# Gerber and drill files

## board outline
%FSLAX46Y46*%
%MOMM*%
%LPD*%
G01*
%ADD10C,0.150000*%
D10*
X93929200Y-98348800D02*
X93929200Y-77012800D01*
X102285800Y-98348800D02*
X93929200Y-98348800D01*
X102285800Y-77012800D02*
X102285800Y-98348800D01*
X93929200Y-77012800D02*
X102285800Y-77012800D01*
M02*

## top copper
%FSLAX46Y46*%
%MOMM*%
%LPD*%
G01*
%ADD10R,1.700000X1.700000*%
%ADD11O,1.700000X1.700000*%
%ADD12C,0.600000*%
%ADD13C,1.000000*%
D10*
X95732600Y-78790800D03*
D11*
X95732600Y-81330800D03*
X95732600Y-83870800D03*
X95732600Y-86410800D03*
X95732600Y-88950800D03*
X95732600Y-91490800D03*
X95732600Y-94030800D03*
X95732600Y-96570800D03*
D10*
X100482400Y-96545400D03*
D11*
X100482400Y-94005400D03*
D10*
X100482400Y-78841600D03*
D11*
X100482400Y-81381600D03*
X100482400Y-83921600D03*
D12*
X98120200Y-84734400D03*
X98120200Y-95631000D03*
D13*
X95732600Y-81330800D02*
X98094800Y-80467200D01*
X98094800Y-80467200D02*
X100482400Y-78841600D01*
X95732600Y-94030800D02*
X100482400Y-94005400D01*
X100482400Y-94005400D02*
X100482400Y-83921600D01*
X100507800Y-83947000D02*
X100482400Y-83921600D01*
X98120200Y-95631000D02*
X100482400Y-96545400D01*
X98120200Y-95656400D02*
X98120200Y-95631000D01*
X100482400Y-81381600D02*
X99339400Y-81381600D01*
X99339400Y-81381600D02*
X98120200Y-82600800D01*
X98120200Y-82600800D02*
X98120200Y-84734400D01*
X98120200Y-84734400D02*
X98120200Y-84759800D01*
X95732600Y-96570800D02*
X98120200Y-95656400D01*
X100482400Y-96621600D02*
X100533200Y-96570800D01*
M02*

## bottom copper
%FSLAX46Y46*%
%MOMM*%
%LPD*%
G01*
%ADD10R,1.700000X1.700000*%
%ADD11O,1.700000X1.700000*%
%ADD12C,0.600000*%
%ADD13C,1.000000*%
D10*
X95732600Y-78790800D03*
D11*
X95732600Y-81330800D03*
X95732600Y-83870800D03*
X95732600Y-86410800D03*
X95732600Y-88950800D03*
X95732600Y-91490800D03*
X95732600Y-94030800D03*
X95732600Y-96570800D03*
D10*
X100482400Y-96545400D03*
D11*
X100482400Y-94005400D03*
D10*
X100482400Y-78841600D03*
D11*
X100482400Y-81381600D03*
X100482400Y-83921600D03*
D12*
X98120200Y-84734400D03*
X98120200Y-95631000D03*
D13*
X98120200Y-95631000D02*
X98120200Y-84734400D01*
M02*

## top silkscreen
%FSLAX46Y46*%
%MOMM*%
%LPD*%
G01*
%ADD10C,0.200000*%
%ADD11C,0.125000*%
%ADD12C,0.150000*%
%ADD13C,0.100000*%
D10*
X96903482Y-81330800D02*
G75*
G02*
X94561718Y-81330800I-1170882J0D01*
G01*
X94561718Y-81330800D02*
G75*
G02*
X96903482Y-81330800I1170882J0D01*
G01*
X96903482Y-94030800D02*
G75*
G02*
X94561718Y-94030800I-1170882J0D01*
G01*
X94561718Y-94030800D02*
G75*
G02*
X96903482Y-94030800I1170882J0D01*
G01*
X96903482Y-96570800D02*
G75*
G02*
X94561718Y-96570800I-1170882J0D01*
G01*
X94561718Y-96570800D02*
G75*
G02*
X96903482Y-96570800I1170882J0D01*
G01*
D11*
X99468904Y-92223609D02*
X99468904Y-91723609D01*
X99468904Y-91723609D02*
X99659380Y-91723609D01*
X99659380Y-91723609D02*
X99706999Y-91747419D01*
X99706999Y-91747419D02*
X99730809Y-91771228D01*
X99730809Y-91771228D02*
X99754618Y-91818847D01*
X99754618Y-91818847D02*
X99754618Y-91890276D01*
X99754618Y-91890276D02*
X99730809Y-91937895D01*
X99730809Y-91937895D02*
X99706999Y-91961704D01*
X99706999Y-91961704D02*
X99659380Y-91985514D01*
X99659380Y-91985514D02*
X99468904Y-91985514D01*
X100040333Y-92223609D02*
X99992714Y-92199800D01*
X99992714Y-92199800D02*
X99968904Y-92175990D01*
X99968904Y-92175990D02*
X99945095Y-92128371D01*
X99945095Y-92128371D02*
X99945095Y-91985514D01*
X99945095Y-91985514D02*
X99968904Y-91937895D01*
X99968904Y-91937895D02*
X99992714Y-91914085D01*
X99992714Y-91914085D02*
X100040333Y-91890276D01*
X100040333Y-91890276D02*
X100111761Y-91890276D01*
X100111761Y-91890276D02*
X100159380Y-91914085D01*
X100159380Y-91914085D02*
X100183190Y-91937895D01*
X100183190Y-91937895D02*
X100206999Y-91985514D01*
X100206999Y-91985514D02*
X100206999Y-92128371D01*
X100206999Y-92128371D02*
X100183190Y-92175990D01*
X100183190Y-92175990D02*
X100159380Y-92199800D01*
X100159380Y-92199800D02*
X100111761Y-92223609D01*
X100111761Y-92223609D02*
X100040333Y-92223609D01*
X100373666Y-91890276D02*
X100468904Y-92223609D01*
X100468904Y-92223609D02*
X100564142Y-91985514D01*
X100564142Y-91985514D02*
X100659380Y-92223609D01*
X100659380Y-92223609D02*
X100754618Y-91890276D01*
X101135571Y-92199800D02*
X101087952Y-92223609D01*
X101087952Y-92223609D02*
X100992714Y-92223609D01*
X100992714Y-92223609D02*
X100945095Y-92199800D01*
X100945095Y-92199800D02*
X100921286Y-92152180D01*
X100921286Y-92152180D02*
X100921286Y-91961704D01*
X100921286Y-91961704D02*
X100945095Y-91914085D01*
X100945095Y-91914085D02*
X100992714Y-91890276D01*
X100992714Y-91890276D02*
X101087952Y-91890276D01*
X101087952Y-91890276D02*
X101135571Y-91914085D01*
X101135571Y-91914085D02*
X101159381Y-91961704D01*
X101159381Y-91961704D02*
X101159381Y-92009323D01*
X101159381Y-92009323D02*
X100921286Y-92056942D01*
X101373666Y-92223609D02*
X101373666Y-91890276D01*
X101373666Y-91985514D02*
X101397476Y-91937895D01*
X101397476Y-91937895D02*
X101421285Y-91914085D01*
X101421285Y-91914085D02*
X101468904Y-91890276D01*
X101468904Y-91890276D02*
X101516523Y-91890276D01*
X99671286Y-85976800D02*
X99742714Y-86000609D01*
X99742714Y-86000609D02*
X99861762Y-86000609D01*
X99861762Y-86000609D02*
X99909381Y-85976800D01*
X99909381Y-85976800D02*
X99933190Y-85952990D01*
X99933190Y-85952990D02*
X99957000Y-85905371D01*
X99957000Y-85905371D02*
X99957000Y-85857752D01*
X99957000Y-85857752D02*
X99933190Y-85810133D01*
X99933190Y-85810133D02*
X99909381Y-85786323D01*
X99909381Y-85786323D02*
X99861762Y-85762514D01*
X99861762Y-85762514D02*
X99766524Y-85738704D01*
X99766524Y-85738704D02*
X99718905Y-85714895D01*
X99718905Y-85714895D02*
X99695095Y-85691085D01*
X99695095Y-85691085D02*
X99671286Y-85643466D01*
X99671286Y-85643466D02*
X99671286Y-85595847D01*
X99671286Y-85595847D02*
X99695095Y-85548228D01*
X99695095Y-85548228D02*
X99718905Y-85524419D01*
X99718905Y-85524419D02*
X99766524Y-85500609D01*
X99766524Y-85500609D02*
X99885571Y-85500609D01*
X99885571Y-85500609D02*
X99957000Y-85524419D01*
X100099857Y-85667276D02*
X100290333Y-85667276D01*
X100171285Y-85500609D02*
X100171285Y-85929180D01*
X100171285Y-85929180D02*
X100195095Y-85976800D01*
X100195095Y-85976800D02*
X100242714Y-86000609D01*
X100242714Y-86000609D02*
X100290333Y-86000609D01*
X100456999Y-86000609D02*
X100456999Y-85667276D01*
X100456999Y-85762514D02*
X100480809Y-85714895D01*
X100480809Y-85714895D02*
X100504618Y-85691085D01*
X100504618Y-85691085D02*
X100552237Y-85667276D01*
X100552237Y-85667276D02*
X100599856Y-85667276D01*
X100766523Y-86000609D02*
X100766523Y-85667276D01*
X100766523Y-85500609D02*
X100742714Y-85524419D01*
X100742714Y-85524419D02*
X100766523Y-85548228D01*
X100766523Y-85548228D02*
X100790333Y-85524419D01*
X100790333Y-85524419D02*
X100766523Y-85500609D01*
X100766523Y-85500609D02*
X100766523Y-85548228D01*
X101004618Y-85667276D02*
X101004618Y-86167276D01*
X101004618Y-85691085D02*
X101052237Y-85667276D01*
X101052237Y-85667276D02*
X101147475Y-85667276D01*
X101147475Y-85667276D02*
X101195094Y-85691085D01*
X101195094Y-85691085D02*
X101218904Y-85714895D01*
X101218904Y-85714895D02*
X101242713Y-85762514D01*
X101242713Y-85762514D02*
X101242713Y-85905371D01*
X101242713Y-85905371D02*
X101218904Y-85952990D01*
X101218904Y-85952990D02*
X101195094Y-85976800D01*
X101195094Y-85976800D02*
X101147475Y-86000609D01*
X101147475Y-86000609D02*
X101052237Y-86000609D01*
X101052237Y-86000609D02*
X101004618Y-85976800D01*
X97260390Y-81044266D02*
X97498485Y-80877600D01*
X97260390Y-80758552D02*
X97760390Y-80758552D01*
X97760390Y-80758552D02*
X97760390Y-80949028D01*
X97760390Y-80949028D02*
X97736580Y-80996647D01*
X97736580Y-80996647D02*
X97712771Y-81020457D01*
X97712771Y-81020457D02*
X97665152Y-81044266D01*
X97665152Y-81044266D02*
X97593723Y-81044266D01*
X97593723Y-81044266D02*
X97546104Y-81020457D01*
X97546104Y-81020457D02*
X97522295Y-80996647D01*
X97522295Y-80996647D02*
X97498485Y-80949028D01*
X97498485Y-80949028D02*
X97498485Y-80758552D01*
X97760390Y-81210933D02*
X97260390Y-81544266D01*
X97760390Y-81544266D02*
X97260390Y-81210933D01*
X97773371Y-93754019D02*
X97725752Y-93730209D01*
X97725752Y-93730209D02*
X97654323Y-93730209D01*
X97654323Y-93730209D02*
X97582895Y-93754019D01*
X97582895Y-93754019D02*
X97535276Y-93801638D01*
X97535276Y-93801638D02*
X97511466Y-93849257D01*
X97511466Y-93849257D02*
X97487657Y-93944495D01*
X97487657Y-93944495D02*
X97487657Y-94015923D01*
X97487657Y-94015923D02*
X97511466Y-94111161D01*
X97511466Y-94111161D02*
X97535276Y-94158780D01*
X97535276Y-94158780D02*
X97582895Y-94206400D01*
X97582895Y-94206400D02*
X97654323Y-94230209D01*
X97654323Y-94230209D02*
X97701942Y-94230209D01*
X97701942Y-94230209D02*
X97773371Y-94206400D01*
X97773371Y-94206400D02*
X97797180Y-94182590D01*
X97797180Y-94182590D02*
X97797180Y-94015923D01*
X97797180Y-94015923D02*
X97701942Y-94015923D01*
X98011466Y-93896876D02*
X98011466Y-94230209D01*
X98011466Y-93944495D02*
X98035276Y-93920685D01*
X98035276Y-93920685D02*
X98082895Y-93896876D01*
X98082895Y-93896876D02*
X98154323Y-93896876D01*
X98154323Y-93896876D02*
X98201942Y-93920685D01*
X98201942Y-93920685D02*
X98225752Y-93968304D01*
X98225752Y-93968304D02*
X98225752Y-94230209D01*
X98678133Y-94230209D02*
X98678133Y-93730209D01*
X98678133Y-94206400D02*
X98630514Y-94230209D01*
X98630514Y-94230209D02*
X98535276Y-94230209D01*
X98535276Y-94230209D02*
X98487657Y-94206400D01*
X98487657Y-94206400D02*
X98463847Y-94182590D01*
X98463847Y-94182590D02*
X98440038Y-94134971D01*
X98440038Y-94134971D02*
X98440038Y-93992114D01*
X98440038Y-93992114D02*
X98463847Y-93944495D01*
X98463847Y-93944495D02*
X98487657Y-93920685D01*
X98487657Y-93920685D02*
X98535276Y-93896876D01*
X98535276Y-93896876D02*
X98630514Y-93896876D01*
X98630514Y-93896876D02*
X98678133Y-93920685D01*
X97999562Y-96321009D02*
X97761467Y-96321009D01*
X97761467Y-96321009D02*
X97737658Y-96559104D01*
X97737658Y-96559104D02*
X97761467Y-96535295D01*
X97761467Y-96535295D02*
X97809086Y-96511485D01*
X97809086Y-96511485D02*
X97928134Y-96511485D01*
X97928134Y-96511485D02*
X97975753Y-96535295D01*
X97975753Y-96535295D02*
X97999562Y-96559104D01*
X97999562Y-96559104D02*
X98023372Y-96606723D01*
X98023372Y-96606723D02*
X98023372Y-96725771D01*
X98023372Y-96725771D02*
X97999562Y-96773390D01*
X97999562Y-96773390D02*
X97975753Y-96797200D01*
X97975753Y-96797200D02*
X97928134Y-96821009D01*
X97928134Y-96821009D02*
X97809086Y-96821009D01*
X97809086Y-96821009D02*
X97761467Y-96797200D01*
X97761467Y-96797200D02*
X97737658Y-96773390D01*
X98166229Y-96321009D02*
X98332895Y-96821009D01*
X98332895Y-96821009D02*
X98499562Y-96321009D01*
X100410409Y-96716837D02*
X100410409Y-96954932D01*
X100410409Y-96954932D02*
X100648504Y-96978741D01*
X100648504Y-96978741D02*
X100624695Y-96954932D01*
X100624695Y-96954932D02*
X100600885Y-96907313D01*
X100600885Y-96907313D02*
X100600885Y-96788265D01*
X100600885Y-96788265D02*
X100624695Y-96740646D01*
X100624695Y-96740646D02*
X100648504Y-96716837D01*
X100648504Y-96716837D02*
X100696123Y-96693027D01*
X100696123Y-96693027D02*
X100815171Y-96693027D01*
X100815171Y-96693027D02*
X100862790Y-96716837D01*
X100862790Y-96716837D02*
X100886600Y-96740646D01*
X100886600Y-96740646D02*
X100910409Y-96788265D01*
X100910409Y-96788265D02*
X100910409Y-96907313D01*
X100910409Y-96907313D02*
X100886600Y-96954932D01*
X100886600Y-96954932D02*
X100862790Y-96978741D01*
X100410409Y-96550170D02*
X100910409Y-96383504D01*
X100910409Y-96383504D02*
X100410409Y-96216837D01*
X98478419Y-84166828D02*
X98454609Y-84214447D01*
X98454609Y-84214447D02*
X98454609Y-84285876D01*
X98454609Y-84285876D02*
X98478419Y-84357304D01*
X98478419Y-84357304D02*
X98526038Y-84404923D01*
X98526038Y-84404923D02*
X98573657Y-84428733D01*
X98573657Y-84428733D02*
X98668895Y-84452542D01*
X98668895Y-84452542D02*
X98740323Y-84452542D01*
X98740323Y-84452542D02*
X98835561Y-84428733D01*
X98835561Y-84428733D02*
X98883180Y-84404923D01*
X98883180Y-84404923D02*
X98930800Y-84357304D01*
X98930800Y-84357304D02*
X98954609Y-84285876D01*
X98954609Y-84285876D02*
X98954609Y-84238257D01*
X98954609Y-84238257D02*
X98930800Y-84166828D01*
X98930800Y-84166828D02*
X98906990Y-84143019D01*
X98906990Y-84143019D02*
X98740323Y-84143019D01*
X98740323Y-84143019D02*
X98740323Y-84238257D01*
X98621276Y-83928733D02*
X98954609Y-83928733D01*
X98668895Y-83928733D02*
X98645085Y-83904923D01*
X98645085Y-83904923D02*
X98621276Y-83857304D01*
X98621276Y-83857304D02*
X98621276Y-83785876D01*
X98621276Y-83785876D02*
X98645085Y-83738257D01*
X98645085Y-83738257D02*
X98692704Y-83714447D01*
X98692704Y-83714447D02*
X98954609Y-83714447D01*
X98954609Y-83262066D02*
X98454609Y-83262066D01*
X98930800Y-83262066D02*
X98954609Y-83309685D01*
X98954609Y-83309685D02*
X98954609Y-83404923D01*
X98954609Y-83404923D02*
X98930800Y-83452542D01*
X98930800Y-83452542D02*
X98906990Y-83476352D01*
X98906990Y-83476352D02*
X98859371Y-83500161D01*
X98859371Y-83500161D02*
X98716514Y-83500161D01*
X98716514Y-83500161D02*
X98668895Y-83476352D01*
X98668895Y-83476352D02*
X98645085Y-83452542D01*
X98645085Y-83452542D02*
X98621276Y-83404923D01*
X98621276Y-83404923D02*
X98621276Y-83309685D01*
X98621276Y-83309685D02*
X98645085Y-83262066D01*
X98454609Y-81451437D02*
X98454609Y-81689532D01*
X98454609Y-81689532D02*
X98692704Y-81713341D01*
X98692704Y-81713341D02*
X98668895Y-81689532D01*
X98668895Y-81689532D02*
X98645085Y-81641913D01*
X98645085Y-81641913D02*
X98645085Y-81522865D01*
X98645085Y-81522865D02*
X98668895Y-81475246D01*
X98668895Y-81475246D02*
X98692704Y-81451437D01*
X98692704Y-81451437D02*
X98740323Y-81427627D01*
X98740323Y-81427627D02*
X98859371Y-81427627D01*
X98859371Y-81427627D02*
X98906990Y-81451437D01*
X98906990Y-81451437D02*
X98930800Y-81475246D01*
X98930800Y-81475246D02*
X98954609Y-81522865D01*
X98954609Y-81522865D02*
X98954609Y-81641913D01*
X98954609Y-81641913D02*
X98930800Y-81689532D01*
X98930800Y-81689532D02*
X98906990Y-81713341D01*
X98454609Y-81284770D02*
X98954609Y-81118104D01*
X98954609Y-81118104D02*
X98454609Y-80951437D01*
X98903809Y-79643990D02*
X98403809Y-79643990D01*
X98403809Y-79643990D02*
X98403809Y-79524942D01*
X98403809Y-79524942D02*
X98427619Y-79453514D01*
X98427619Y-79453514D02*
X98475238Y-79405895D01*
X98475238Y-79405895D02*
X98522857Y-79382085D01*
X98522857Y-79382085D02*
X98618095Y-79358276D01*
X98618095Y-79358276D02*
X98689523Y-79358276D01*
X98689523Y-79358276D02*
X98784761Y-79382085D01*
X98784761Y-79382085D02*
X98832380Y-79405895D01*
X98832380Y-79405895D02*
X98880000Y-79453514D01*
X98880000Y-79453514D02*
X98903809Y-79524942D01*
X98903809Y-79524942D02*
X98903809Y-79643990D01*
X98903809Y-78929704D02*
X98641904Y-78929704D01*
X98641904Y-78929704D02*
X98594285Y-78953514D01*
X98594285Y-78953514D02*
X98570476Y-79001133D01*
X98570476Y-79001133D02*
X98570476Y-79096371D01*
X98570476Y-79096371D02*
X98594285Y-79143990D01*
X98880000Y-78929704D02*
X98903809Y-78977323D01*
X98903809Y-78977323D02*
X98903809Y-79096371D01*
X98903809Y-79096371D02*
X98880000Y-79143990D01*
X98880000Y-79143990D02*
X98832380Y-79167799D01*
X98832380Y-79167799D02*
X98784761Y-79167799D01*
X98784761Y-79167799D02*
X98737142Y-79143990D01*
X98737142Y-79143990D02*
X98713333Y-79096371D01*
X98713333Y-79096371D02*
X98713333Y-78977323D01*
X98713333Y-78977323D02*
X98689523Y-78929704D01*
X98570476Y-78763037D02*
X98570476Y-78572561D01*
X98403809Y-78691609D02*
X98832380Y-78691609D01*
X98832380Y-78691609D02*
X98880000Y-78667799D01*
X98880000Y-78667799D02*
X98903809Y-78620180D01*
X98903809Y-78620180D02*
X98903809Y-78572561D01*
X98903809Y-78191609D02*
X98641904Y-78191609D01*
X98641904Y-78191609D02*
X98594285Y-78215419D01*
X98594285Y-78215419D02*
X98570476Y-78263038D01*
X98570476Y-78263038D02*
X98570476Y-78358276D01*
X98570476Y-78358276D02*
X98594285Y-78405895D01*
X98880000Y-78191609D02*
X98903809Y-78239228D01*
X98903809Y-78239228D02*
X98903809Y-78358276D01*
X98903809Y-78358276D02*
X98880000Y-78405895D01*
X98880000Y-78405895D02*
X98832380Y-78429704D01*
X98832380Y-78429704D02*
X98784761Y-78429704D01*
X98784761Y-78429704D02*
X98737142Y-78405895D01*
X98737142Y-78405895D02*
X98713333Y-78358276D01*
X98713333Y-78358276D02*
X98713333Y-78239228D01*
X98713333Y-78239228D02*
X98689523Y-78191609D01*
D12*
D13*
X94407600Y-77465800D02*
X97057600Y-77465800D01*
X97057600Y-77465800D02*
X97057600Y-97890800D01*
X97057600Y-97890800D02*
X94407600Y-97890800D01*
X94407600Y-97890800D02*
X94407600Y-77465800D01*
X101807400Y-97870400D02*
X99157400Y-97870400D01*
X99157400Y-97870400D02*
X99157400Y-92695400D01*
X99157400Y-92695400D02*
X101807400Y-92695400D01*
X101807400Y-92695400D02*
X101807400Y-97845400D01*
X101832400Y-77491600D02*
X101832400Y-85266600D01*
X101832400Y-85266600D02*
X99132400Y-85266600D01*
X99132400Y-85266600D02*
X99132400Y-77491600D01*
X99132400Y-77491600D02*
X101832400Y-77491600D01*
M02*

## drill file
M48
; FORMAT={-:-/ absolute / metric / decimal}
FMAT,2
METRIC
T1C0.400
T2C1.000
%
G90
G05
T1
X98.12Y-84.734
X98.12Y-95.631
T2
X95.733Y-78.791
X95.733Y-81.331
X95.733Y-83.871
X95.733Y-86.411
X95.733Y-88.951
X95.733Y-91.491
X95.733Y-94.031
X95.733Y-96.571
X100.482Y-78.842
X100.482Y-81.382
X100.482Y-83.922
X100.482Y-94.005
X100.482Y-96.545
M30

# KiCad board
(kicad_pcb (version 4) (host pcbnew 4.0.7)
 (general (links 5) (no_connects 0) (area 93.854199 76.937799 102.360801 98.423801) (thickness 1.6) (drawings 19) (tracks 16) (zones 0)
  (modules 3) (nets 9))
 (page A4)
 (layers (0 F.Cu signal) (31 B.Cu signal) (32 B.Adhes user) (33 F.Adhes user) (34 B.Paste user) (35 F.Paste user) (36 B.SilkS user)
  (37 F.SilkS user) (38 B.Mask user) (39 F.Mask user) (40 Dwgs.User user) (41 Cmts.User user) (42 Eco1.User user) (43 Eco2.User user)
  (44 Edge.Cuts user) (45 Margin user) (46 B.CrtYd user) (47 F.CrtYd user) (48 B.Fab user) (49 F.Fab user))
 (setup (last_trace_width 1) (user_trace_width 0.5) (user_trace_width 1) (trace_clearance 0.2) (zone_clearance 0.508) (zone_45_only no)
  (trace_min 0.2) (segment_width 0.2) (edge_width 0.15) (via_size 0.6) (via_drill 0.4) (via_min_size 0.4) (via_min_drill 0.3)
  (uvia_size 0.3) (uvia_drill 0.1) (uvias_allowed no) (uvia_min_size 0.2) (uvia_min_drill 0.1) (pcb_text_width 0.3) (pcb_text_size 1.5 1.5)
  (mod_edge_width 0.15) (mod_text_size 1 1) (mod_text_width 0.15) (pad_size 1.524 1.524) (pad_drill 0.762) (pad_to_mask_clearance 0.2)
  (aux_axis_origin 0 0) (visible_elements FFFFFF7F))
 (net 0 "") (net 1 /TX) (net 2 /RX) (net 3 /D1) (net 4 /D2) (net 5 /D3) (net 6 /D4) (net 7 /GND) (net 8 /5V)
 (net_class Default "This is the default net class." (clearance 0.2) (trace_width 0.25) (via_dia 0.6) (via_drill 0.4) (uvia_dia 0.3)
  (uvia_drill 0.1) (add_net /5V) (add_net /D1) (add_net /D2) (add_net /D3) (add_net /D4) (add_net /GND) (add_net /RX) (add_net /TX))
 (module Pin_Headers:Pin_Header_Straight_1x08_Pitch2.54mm (layer F.Cu) (at 95.7326 78.7908)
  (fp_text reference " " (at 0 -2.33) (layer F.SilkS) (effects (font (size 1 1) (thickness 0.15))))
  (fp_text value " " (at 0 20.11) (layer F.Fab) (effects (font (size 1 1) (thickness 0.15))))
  (fp_line (start -1.325 -1.325) (end 1.325 -1.325) (layer F.SilkS) (width 0.1))
  (fp_line (start 1.325 -1.325) (end 1.325 19.1) (layer F.SilkS) (width 0.1))
  (fp_line (start 1.325 19.1) (end -1.325 19.1) (layer F.SilkS) (width 0.1))
  (fp_line (start -1.325 19.1) (end -1.325 -1.325) (layer F.SilkS) (width 0.1))
  (pad 1 thru_hole rect (at 0 0) (size 1.7 1.7) (drill 1) (layers *.Cu *.Mask) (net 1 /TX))
  (pad 2 thru_hole oval (at 0 2.54) (size 1.7 1.7) (drill 1) (layers *.Cu *.Mask) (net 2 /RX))
  (pad 3 thru_hole oval (at 0 5.08) (size 1.7 1.7) (drill 1) (layers *.Cu *.Mask) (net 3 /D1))
  (pad 4 thru_hole oval (at 0 7.62) (size 1.7 1.7) (drill 1) (layers *.Cu *.Mask) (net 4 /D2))
  (pad 5 thru_hole oval (at 0 10.16) (size 1.7 1.7) (drill 1) (layers *.Cu *.Mask) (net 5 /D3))
  (pad 6 thru_hole oval (at 0 12.7) (size 1.7 1.7) (drill 1) (layers *.Cu *.Mask) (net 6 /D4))
  (pad 7 thru_hole oval (at 0 15.24) (size 1.7 1.7) (drill 1) (layers *.Cu *.Mask) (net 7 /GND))
  (pad 8 thru_hole oval (at 0 17.78) (size 1.7 1.7) (drill 1) (layers *.Cu *.Mask) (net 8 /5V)))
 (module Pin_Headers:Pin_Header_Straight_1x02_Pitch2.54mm (layer F.Cu) (at 100.4824 96.5454 180)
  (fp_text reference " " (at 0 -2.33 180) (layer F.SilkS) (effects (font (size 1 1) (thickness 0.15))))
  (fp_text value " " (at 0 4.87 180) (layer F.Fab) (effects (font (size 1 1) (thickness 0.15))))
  (fp_line (start -1.325 -1.325) (end 1.325 -1.325) (layer F.SilkS) (width 0.1))
  (fp_line (start 1.325 -1.325) (end 1.325 3.85) (layer F.SilkS) (width 0.1))
  (fp_line (start 1.325 3.85) (end -1.325 3.85) (layer F.SilkS) (width 0.1))
  (fp_line (start -1.325 3.85) (end -1.325 -1.3) (layer F.SilkS) (width 0.1))
  (pad 1 thru_hole rect (at 0 0 180) (size 1.7 1.7) (drill 1) (layers *.Cu *.Mask) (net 8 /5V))
  (pad 2 thru_hole oval (at 0 2.54 180) (size 1.7 1.7) (drill 1) (layers *.Cu *.Mask) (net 7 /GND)))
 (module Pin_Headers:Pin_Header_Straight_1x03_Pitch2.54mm (layer F.Cu) (at 100.4824 78.8416)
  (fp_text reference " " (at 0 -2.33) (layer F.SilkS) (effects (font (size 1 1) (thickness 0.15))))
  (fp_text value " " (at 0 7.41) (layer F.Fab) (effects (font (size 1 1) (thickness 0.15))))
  (fp_line (start 1.35 -1.35) (end 1.35 6.425) (layer F.SilkS) (width 0.1))
  (fp_line (start 1.35 6.425) (end -1.35 6.425) (layer F.SilkS) (width 0.1))
  (fp_line (start -1.35 6.425) (end -1.35 -1.35) (layer F.SilkS) (width 0.1))
  (fp_line (start -1.35 -1.35) (end 1.35 -1.35) (layer F.SilkS) (width 0.1))
  (pad 1 thru_hole rect (at 0 0) (size 1.7 1.7) (drill 1) (layers *.Cu *.Mask) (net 2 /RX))
  (pad 2 thru_hole oval (at 0 2.54) (size 1.7 1.7) (drill 1) (layers *.Cu *.Mask) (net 8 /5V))
  (pad 3 thru_hole oval (at 0 5.08) (size 1.7 1.7) (drill 1) (layers *.Cu *.Mask) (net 7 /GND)))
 (gr_circle (center 95.7326 81.3308) (end 96.4946 82.2198) (layer F.SilkS) (width 0.2))
 (gr_circle (center 95.7326 94.0308) (end 96.4946 94.9198) (layer F.SilkS) (width 0.2))
 (gr_circle (center 95.7326 96.5708) (end 96.4946 97.4598) (layer F.SilkS) (width 0.2))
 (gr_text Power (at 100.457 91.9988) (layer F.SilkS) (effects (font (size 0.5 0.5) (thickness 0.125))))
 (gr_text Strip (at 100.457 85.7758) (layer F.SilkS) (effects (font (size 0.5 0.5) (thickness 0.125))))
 (gr_line (start 93.9292 98.3488) (end 93.9292 77.0128) (angle 90) (layer Edge.Cuts) (width 0.15))
 (gr_line (start 102.2858 98.3488) (end 93.9292 98.3488) (angle 90) (layer Edge.Cuts) (width 0.15))
 (gr_line (start 102.2858 77.0128) (end 102.2858 98.3488) (angle 90) (layer Edge.Cuts) (width 0.15))
 (gr_line (start 93.9292 77.0128) (end 102.2858 77.0128) (angle 90) (layer Edge.Cuts) (width 0.15))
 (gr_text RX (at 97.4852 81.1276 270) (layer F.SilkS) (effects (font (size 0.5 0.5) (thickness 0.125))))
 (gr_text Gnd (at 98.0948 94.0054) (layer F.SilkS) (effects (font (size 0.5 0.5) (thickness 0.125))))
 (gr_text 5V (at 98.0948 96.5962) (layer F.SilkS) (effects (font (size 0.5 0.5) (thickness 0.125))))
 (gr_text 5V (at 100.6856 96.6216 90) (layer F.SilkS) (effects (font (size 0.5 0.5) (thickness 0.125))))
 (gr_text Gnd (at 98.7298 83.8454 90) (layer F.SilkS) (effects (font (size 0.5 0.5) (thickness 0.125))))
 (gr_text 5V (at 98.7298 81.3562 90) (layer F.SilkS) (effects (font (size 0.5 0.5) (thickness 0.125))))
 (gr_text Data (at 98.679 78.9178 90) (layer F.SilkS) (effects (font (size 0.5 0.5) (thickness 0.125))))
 (segment (start 95.7326 81.3308) (end 98.0948 80.4672) (width 1) (layer F.Cu) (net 2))
 (segment (start 98.0948 80.4672) (end 100.4824 78.8416) (width 1) (layer F.Cu) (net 2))
 (segment (start 95.7326 94.0308) (end 100.4824 94.0054) (width 1) (layer F.Cu) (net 7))
 (segment (start 100.4824 94.0054) (end 100.4824 83.9216) (width 1) (layer F.Cu) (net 7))
 (segment (start 100.5078 83.947) (end 100.4824 83.9216) (width 1) (layer F.Cu) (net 7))
 (segment (start 98.1202 95.631) (end 100.4824 96.5454) (width 1) (layer F.Cu) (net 8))
 (via (at 98.1202 84.7344) (size 0.6) (drill 0.4) (layers F.Cu B.Cu) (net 8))
 (segment (start 98.1202 95.6564) (end 98.1202 95.631) (width 1) (layer F.Cu) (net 8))
 (via (at 98.1202 95.631) (size 0.6) (drill 0.4) (layers F.Cu B.Cu) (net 8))
 (segment (start 98.1202 95.631) (end 98.1202 84.7344) (width 1) (layer B.Cu) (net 8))
 (segment (start 100.4824 81.3816) (end 99.3394 81.3816) (width 1) (layer F.Cu) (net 8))
 (segment (start 99.3394 81.3816) (end 98.1202 82.6008) (width 1) (layer F.Cu) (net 8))
 (segment (start 98.1202 82.6008) (end 98.1202 84.7344) (width 1) (layer F.Cu) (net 8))
 (segment (start 98.1202 84.7344) (end 98.1202 84.7598) (width 1) (layer F.Cu) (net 8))
 (segment (start 95.7326 96.5708) (end 98.1202 95.6564) (width 1) (layer F.Cu) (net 8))
 (segment (start 100.4824 96.6216) (end 100.5332 96.5708) (width 1) (layer F.Cu) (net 8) (status 30)))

